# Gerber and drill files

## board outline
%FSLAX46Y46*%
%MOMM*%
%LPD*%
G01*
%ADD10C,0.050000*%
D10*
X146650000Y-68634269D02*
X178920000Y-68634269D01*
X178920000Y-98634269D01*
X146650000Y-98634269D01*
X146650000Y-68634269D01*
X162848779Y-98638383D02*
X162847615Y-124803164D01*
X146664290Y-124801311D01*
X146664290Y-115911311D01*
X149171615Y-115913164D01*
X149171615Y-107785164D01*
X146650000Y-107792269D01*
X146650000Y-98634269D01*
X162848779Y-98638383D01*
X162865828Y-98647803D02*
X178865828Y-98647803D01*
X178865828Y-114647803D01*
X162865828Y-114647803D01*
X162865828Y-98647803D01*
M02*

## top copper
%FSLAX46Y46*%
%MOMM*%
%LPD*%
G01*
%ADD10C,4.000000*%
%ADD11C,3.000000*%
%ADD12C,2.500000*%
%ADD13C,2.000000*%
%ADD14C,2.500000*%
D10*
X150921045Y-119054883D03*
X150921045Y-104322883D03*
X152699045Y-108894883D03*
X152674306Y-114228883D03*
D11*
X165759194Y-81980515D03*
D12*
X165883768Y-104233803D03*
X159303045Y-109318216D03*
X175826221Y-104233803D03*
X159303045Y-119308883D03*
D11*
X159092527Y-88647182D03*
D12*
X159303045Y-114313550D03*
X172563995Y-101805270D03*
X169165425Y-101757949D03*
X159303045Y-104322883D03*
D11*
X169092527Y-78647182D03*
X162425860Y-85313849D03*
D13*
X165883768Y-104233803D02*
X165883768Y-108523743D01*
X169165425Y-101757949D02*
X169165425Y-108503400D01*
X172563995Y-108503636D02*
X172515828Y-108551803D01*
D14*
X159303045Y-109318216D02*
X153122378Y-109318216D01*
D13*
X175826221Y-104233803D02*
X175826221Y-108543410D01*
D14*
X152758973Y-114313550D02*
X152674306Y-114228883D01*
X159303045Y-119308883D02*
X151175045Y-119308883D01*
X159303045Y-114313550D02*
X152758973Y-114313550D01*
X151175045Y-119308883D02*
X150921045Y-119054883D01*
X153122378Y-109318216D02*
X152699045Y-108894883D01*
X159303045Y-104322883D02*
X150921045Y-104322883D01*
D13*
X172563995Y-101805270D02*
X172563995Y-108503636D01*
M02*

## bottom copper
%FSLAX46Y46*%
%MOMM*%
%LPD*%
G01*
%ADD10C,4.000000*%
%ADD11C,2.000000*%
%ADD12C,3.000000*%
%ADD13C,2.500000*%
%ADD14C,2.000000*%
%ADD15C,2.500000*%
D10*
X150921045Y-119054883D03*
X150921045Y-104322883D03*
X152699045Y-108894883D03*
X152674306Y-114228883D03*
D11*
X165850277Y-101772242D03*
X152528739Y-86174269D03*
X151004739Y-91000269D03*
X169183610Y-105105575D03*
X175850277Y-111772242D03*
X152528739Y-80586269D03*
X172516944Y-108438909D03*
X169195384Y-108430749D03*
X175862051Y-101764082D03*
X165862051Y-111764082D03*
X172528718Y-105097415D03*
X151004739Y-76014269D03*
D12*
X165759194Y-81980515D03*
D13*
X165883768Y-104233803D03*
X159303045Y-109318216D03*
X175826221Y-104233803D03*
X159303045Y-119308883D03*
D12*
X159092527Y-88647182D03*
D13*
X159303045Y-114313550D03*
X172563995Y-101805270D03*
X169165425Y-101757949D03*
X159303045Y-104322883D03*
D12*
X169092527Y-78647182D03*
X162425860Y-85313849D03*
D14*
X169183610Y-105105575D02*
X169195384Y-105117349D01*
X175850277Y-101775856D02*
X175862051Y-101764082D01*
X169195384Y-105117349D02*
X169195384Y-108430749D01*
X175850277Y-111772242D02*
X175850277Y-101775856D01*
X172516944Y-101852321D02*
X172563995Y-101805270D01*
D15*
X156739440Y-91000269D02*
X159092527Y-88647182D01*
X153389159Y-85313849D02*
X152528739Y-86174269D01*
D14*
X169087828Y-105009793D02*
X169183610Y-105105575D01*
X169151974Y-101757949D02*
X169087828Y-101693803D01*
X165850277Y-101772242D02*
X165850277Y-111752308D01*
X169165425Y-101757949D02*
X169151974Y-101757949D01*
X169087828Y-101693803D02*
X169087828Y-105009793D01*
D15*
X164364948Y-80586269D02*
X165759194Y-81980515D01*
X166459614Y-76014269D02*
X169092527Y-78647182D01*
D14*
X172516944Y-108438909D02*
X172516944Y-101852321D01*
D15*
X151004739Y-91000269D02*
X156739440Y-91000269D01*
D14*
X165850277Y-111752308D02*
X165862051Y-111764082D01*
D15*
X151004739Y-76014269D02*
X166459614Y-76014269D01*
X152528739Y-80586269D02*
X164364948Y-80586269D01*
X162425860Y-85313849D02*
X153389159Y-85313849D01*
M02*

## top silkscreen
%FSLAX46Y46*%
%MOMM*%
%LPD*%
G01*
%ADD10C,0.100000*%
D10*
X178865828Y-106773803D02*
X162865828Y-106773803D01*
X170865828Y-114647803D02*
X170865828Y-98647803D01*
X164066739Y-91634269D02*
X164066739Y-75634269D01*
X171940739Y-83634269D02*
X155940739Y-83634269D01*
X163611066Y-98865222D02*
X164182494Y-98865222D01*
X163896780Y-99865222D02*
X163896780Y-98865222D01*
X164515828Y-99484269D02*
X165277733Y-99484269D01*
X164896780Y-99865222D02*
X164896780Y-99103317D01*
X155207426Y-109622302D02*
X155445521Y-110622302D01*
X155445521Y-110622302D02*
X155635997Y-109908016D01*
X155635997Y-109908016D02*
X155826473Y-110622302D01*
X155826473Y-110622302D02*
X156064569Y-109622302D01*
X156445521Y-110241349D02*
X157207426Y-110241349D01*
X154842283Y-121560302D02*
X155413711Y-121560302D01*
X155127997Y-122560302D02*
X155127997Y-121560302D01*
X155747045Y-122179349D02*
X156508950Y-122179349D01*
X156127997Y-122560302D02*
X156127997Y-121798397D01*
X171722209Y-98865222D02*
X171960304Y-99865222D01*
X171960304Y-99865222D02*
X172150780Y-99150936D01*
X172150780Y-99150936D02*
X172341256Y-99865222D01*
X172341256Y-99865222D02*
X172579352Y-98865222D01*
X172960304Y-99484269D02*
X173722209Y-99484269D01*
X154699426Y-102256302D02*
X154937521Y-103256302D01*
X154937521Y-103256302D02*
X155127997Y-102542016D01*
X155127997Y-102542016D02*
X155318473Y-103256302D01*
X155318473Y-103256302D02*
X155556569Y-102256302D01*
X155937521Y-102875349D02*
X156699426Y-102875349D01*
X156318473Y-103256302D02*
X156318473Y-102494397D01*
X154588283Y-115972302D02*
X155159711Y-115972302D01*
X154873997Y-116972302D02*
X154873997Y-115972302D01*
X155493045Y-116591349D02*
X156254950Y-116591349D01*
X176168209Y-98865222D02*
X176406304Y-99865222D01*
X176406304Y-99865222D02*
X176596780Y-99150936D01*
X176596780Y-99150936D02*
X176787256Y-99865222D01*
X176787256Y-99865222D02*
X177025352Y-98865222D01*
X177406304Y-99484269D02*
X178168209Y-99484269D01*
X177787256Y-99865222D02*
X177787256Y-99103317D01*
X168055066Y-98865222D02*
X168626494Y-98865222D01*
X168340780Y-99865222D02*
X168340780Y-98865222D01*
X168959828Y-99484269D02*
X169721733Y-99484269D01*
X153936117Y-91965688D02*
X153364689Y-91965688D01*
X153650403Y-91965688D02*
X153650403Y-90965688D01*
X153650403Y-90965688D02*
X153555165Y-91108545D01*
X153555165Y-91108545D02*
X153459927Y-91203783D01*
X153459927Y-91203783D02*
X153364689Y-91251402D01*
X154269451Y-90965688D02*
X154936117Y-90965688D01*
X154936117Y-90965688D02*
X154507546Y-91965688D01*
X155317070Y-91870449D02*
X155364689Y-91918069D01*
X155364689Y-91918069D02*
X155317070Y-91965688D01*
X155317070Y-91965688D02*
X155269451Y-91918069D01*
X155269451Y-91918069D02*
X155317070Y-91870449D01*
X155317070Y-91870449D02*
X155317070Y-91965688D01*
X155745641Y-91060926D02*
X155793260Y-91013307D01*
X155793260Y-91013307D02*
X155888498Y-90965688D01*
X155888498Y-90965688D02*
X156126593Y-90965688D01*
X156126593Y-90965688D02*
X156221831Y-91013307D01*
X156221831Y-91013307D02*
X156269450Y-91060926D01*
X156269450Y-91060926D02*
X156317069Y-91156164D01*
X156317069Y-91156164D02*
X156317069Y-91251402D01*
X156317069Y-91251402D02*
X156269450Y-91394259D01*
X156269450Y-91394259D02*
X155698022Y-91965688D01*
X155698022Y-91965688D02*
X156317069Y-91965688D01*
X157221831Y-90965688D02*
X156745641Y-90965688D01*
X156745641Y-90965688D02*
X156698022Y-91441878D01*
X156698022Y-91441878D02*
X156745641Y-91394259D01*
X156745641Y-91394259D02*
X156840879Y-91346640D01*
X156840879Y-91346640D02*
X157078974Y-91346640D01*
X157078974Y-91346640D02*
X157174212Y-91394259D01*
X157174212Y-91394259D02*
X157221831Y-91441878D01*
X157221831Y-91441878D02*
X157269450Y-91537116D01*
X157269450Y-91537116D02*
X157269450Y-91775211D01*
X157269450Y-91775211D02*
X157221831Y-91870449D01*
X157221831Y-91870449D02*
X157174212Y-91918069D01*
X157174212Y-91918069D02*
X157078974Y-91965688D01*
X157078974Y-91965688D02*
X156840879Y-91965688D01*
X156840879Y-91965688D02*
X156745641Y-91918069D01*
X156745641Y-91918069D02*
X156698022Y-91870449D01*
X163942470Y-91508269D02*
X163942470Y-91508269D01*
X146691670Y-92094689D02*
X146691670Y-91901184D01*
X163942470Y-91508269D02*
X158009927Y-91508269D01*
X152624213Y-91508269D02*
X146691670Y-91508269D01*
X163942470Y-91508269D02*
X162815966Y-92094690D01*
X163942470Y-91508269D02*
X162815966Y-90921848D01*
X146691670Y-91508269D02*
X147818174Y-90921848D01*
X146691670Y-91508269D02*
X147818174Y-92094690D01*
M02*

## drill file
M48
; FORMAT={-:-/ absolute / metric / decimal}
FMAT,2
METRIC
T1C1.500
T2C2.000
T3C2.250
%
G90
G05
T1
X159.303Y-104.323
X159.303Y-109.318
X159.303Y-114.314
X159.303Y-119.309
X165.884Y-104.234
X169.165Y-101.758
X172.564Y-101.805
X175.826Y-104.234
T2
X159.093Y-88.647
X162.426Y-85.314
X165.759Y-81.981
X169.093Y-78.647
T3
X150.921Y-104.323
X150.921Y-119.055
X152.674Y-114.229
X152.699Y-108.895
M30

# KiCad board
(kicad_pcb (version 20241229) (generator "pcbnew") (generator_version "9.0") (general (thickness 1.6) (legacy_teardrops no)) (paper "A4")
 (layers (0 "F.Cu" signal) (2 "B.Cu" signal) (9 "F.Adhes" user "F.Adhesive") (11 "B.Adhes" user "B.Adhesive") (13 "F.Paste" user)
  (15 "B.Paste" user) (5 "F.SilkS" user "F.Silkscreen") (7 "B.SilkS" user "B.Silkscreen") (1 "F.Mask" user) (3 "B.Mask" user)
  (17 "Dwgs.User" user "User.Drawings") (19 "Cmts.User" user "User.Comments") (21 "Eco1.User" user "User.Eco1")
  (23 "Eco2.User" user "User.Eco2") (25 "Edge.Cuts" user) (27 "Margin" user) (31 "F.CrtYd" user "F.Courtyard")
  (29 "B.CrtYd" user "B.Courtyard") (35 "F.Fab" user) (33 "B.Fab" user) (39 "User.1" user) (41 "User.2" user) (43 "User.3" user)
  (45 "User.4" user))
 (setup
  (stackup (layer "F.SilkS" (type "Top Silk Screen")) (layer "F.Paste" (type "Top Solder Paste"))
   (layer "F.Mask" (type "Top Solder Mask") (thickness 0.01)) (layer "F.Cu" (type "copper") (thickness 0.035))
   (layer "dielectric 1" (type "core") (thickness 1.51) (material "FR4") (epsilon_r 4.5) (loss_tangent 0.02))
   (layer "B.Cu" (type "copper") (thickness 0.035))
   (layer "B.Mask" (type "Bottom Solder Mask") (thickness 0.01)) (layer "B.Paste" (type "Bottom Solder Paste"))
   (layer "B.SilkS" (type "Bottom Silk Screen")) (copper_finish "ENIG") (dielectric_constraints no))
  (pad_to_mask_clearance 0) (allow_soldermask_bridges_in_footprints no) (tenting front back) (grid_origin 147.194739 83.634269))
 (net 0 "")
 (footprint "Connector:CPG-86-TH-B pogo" (layer "F.Cu") (at 150.921045 119.054883)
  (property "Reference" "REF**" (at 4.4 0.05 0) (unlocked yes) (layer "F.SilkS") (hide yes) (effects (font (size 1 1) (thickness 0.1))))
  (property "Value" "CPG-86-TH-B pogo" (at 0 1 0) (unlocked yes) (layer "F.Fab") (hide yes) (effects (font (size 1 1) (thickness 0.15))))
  (pad "1" thru_hole circle (at 0 0) (size 4 4) (drill 2.25) (layers "*.Cu" "*.Mask") (remove_unused_layers no)))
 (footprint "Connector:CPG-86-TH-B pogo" (layer "F.Cu") (at 150.921045 104.322883)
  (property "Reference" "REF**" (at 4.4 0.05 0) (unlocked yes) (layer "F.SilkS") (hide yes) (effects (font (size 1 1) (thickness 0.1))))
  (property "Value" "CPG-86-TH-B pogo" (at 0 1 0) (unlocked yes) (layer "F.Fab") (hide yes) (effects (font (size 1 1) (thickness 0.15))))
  (pad "1" thru_hole circle (at 0 0) (size 4 4) (drill 2.25) (layers "*.Cu" "*.Mask") (remove_unused_layers no)))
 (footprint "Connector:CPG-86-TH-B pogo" (layer "F.Cu") (at 152.699045 108.894883)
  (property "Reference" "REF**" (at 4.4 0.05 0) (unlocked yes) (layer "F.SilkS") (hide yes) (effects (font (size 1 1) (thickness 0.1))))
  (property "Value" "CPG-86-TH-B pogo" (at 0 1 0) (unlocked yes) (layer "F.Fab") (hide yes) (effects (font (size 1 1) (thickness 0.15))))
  (pad "1" thru_hole circle (at 0 0) (size 4 4) (drill 2.25) (layers "*.Cu" "*.Mask") (remove_unused_layers no)))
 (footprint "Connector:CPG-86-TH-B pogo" (layer "F.Cu") (at 152.674306 114.228883)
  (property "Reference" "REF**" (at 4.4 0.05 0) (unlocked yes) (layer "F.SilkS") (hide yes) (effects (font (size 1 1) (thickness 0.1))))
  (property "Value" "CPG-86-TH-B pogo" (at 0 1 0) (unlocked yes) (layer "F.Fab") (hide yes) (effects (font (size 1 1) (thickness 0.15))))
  (pad "1" thru_hole circle (at 0 0) (size 4 4) (drill 2.25) (layers "*.Cu" "*.Mask") (remove_unused_layers no)))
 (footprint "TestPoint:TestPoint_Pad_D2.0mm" (layer "B.Cu") (at 165.850277 101.772242 180)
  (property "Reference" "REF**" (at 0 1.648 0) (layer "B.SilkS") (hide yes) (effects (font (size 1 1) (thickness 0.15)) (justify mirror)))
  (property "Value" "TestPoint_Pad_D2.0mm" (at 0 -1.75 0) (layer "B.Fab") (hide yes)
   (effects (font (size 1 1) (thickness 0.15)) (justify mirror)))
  (pad "1" smd circle (at 0 0 180) (size 2 2) (layers "B.Cu" "B.Mask")))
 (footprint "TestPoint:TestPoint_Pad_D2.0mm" (layer "B.Cu") (at 152.528739 86.174269 180)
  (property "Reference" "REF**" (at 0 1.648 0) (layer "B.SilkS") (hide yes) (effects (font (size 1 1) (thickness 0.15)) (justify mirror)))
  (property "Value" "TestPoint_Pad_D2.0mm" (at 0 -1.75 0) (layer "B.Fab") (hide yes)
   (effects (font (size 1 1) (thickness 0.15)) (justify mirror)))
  (pad "1" smd circle (at 0 0 180) (size 2 2) (layers "B.Cu" "B.Mask")))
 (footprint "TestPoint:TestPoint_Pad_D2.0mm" (layer "B.Cu") (at 151.004739 91.000269 180)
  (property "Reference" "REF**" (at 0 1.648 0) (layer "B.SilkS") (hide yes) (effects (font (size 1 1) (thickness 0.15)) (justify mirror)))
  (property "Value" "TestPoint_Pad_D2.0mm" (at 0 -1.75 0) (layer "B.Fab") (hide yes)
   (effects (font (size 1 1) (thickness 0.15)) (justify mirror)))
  (pad "1" smd circle (at 0 0 180) (size 2 2) (layers "B.Cu" "B.Mask")))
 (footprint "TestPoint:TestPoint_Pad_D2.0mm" (layer "B.Cu") (at 169.18361 105.105575 180)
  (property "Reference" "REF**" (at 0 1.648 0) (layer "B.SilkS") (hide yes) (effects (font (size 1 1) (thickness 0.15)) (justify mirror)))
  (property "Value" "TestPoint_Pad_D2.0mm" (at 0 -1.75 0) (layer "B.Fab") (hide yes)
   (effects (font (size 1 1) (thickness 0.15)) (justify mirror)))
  (pad "1" smd circle (at 0 0 180) (size 2 2) (layers "B.Cu" "B.Mask")))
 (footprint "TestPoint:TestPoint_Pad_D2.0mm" (layer "B.Cu") (at 175.850277 111.772242 180)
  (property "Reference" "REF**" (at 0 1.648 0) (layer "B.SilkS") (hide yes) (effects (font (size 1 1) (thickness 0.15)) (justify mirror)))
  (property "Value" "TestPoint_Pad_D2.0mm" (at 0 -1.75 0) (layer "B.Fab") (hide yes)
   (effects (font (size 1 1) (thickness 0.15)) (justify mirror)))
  (pad "1" smd circle (at 0 0 180) (size 2 2) (layers "B.Cu" "B.Mask")))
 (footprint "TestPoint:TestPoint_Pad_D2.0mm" (layer "B.Cu") (at 152.528739 80.586269 180)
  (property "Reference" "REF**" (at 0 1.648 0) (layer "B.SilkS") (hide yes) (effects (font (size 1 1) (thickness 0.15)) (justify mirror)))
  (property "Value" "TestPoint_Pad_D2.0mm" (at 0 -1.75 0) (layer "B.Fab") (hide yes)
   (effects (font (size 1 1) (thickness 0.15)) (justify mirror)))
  (pad "1" smd circle (at 0 0 180) (size 2 2) (layers "B.Cu" "B.Mask")))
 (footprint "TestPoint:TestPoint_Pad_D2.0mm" (layer "B.Cu") (at 172.516944 108.438909 180)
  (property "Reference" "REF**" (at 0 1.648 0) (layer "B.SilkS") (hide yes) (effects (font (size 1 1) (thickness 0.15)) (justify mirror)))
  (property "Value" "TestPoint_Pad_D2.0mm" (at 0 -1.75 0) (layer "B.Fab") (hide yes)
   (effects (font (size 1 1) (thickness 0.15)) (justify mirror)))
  (pad "1" smd circle (at 0 0 180) (size 2 2) (layers "B.Cu" "B.Mask")))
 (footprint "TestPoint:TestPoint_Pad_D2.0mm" (layer "B.Cu") (at 169.195384 108.430749 90)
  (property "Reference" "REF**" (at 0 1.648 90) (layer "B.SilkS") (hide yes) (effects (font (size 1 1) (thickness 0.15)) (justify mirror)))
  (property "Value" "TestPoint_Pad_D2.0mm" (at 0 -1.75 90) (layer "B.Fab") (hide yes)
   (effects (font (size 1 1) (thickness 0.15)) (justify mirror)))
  (pad "1" smd circle (at 0 0 90) (size 2 2) (layers "B.Cu" "B.Mask")))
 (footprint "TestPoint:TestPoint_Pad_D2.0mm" (layer "B.Cu") (at 175.862051 101.764082 90)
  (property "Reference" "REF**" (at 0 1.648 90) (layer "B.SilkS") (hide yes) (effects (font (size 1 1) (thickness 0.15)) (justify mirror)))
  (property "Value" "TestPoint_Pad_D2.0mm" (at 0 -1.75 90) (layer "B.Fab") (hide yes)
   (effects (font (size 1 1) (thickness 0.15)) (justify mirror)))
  (pad "1" smd circle (at 0 0 90) (size 2 2) (layers "B.Cu" "B.Mask")))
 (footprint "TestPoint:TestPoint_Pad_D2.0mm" (layer "B.Cu") (at 165.862051 111.764082 90)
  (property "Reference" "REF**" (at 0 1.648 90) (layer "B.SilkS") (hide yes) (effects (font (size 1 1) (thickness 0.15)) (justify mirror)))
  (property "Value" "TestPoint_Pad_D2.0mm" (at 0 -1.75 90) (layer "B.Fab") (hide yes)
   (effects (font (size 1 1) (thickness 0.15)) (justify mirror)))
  (pad "1" smd circle (at 0 0 90) (size 2 2) (layers "B.Cu" "B.Mask")))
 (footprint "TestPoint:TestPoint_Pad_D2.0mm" (layer "B.Cu") (at 172.528718 105.097415 90)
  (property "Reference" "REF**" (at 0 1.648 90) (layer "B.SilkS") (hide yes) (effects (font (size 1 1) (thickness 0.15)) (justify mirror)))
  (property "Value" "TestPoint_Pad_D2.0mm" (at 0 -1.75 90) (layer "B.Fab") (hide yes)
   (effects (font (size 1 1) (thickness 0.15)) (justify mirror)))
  (pad "1" smd circle (at 0 0 90) (size 2 2) (layers "B.Cu" "B.Mask")))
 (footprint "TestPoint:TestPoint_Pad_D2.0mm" (layer "B.Cu") (at 151.004739 76.014269 180)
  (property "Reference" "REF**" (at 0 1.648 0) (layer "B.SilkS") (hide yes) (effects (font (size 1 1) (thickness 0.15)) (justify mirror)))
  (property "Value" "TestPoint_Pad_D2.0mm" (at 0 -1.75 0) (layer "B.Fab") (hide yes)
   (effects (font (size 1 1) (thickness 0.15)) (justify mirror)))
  (pad "1" smd circle (at 0 0 180) (size 2 2) (layers "B.Cu" "B.Mask")))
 (gr_line (start 178.865828 106.773803) (end 162.865828 106.773803) (stroke (width 0.1) (type solid)) (layer "F.SilkS"))
 (gr_line (start 170.865828 114.647803) (end 170.865828 98.647803) (stroke (width 0.1) (type solid)) (layer "F.SilkS"))
 (gr_line (start 164.066739 91.634269) (end 164.066739 75.634269) (stroke (width 0.1) (type solid)) (layer "F.SilkS"))
 (gr_line (start 171.940739 83.634269) (end 155.940739 83.634269) (stroke (width 0.1) (type solid)) (layer "F.SilkS"))
 (gr_rect (start 146.65 68.634269) (end 178.92 98.634269) (stroke (width 0.05) (type solid)) (fill no) (layer "Edge.Cuts"))
 (gr_poly
  (pts (xy 162.848779 98.638383) (xy 162.847615 124.803164) (xy 146.66429 124.801311) (xy 146.66429 115.911311) (xy 149.171615 115.913164)
   (xy 149.171615 107.785164) (xy 146.65 107.792269) (xy 146.65 98.634269))
  (stroke (width 0.05) (type solid)) (fill no) (layer "Edge.Cuts"))
 (gr_rect (start 162.865828 98.647803) (end 178.865828 114.647803) (stroke (width 0.05) (type solid)) (fill no) (layer "Edge.Cuts"))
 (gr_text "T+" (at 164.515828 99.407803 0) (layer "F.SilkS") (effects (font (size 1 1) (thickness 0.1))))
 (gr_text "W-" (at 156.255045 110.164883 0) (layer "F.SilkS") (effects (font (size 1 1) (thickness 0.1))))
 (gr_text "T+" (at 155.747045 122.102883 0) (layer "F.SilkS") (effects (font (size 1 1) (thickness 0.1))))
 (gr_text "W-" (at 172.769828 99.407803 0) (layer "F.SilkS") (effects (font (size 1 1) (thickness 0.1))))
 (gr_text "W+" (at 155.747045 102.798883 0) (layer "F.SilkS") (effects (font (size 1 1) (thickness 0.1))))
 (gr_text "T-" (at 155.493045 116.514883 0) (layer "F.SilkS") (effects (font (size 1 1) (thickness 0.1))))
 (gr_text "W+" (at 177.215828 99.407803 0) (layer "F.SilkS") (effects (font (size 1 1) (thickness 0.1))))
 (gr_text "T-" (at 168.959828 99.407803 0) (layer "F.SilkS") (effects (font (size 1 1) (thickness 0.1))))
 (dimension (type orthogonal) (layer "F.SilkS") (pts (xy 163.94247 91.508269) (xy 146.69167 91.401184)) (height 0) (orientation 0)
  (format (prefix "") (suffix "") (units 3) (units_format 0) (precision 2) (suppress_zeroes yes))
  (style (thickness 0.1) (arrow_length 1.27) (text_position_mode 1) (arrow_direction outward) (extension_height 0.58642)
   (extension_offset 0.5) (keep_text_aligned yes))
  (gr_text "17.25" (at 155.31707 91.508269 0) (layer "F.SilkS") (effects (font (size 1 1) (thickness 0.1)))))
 (segment (start 165.883768 104.233803) (end 165.883768 108.523743) (width 2) (layers "F.Cu" "F.Mask") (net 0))
 (segment (start 169.165425 101.757949) (end 169.165425 108.5034) (width 2) (layers "F.Cu" "F.Mask") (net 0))
 (segment (start 172.563995 108.503636) (end 172.515828 108.551803) (width 2) (layer "F.Cu") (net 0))
 (segment (start 159.303045 109.318216) (end 153.122378 109.318216) (width 2.5) (layer "F.Cu") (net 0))
 (segment (start 175.826221 104.233803) (end 175.826221 108.54341) (width 2) (layers "F.Cu" "F.Mask") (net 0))
 (segment (start 152.758973 114.31355) (end 152.674306 114.228883) (width 2.5) (layer "F.Cu") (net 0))
 (segment (start 159.303045 119.308883) (end 151.175045 119.308883) (width 2.5) (layer "F.Cu") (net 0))
 (segment (start 159.303045 114.31355) (end 152.758973 114.31355) (width 2.5) (layer "F.Cu") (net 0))
 (segment (start 151.175045 119.308883) (end 150.921045 119.054883) (width 2.5) (layer "F.Cu") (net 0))
 (segment (start 153.122378 109.318216) (end 152.699045 108.894883) (width 2.5) (layer "F.Cu") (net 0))
 (segment (start 159.303045 104.322883) (end 150.921045 104.322883) (width 2.5) (layer "F.Cu") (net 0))
 (segment (start 172.563995 101.80527) (end 172.563995 108.503636) (width 2) (layers "F.Cu" "F.Mask") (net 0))
 (via (at 165.759194 81.980515) (size 3) (drill 2) (layers "F.Cu" "B.Cu") (tenting none) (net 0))
 (via (at 165.883768 104.233803) (size 2.5) (drill 1.5) (layers "F.Cu" "B.Cu") (tenting none) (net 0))
 (via (at 159.303045 109.318216) (size 2.5) (drill 1.5) (layers "F.Cu" "B.Cu") (tenting none) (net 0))
 (via (at 175.826221 104.233803) (size 2.5) (drill 1.5) (layers "F.Cu" "B.Cu") (tenting none) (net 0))
 (via (at 159.303045 119.308883) (size 2.5) (drill 1.5) (layers "F.Cu" "B.Cu") (tenting none) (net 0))
 (via (at 159.092527 88.647182) (size 3) (drill 2) (layers "F.Cu" "B.Cu") (tenting none) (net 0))
 (via (at 159.303045 114.31355) (size 2.5) (drill 1.5) (layers "F.Cu" "B.Cu") (tenting none) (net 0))
 (via (at 172.563995 101.80527) (size 2.5) (drill 1.5) (layers "F.Cu" "B.Cu") (tenting none) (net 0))
 (via (at 169.165425 101.757949) (size 2.5) (drill 1.5) (layers "F.Cu" "B.Cu") (tenting none) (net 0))
 (via (at 159.303045 104.322883) (size 2.5) (drill 1.5) (layers "F.Cu" "B.Cu") (tenting none) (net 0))
 (via (at 169.092527 78.647182) (size 3) (drill 2) (layers "F.Cu" "B.Cu") (tenting none) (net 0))
 (via (at 162.42586 85.313849) (size 3) (drill 2) (layers "F.Cu" "B.Cu") (tenting none) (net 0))
 (segment (start 169.18361 105.105575) (end 169.195384 105.117349) (width 2) (layer "B.Cu") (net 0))
 (segment (start 175.850277 101.775856) (end 175.862051 101.764082) (width 2) (layer "B.Cu") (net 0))
 (segment (start 169.195384 105.117349) (end 169.195384 108.430749) (width 2) (layer "B.Cu") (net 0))
 (segment (start 175.850277 111.772242) (end 175.850277 101.775856) (width 2) (layer "B.Cu") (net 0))
 (segment (start 172.516944 101.852321) (end 172.563995 101.80527) (width 2) (layer "B.Cu") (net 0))
 (segment (start 156.73944 91.000269) (end 159.092527 88.647182) (width 2.5) (layer "B.Cu") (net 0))
 (segment (start 153.389159 85.313849) (end 152.528739 86.174269) (width 2.5) (layer "B.Cu") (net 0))
 (segment (start 169.087828 105.009793) (end 169.18361 105.105575) (width 2) (layer "B.Cu") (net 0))
 (segment (start 169.151974 101.757949) (end 169.087828 101.693803) (width 2) (layer "B.Cu") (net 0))
 (segment (start 165.850277 101.772242) (end 165.850277 111.752308) (width 2) (layer "B.Cu") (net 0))
 (segment (start 169.165425 101.757949) (end 169.151974 101.757949) (width 2) (layer "B.Cu") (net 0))
 (segment (start 169.087828 101.693803) (end 169.087828 105.009793) (width 2) (layer "B.Cu") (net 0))
 (segment (start 164.364948 80.586269) (end 165.759194 81.980515) (width 2.5) (layer "B.Cu") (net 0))
 (segment (start 166.459614 76.014269) (end 169.092527 78.647182) (width 2.5) (layer "B.Cu") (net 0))
 (segment (start 172.516944 108.438909) (end 172.516944 101.852321) (width 2) (layer "B.Cu") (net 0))
 (segment (start 151.004739 91.000269) (end 156.73944 91.000269) (width 2.5) (layer "B.Cu") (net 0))
 (segment (start 165.850277 111.752308) (end 165.862051 111.764082) (width 2) (layer "B.Cu") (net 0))
 (segment (start 151.004739 76.014269) (end 166.459614 76.014269) (width 2.5) (layer "B.Cu") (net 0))
 (segment (start 152.528739 80.586269) (end 164.364948 80.586269) (width 2.5) (layer "B.Cu") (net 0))
 (segment (start 162.42586 85.313849) (end 153.389159 85.313849) (width 2.5) (layer "B.Cu") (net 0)))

